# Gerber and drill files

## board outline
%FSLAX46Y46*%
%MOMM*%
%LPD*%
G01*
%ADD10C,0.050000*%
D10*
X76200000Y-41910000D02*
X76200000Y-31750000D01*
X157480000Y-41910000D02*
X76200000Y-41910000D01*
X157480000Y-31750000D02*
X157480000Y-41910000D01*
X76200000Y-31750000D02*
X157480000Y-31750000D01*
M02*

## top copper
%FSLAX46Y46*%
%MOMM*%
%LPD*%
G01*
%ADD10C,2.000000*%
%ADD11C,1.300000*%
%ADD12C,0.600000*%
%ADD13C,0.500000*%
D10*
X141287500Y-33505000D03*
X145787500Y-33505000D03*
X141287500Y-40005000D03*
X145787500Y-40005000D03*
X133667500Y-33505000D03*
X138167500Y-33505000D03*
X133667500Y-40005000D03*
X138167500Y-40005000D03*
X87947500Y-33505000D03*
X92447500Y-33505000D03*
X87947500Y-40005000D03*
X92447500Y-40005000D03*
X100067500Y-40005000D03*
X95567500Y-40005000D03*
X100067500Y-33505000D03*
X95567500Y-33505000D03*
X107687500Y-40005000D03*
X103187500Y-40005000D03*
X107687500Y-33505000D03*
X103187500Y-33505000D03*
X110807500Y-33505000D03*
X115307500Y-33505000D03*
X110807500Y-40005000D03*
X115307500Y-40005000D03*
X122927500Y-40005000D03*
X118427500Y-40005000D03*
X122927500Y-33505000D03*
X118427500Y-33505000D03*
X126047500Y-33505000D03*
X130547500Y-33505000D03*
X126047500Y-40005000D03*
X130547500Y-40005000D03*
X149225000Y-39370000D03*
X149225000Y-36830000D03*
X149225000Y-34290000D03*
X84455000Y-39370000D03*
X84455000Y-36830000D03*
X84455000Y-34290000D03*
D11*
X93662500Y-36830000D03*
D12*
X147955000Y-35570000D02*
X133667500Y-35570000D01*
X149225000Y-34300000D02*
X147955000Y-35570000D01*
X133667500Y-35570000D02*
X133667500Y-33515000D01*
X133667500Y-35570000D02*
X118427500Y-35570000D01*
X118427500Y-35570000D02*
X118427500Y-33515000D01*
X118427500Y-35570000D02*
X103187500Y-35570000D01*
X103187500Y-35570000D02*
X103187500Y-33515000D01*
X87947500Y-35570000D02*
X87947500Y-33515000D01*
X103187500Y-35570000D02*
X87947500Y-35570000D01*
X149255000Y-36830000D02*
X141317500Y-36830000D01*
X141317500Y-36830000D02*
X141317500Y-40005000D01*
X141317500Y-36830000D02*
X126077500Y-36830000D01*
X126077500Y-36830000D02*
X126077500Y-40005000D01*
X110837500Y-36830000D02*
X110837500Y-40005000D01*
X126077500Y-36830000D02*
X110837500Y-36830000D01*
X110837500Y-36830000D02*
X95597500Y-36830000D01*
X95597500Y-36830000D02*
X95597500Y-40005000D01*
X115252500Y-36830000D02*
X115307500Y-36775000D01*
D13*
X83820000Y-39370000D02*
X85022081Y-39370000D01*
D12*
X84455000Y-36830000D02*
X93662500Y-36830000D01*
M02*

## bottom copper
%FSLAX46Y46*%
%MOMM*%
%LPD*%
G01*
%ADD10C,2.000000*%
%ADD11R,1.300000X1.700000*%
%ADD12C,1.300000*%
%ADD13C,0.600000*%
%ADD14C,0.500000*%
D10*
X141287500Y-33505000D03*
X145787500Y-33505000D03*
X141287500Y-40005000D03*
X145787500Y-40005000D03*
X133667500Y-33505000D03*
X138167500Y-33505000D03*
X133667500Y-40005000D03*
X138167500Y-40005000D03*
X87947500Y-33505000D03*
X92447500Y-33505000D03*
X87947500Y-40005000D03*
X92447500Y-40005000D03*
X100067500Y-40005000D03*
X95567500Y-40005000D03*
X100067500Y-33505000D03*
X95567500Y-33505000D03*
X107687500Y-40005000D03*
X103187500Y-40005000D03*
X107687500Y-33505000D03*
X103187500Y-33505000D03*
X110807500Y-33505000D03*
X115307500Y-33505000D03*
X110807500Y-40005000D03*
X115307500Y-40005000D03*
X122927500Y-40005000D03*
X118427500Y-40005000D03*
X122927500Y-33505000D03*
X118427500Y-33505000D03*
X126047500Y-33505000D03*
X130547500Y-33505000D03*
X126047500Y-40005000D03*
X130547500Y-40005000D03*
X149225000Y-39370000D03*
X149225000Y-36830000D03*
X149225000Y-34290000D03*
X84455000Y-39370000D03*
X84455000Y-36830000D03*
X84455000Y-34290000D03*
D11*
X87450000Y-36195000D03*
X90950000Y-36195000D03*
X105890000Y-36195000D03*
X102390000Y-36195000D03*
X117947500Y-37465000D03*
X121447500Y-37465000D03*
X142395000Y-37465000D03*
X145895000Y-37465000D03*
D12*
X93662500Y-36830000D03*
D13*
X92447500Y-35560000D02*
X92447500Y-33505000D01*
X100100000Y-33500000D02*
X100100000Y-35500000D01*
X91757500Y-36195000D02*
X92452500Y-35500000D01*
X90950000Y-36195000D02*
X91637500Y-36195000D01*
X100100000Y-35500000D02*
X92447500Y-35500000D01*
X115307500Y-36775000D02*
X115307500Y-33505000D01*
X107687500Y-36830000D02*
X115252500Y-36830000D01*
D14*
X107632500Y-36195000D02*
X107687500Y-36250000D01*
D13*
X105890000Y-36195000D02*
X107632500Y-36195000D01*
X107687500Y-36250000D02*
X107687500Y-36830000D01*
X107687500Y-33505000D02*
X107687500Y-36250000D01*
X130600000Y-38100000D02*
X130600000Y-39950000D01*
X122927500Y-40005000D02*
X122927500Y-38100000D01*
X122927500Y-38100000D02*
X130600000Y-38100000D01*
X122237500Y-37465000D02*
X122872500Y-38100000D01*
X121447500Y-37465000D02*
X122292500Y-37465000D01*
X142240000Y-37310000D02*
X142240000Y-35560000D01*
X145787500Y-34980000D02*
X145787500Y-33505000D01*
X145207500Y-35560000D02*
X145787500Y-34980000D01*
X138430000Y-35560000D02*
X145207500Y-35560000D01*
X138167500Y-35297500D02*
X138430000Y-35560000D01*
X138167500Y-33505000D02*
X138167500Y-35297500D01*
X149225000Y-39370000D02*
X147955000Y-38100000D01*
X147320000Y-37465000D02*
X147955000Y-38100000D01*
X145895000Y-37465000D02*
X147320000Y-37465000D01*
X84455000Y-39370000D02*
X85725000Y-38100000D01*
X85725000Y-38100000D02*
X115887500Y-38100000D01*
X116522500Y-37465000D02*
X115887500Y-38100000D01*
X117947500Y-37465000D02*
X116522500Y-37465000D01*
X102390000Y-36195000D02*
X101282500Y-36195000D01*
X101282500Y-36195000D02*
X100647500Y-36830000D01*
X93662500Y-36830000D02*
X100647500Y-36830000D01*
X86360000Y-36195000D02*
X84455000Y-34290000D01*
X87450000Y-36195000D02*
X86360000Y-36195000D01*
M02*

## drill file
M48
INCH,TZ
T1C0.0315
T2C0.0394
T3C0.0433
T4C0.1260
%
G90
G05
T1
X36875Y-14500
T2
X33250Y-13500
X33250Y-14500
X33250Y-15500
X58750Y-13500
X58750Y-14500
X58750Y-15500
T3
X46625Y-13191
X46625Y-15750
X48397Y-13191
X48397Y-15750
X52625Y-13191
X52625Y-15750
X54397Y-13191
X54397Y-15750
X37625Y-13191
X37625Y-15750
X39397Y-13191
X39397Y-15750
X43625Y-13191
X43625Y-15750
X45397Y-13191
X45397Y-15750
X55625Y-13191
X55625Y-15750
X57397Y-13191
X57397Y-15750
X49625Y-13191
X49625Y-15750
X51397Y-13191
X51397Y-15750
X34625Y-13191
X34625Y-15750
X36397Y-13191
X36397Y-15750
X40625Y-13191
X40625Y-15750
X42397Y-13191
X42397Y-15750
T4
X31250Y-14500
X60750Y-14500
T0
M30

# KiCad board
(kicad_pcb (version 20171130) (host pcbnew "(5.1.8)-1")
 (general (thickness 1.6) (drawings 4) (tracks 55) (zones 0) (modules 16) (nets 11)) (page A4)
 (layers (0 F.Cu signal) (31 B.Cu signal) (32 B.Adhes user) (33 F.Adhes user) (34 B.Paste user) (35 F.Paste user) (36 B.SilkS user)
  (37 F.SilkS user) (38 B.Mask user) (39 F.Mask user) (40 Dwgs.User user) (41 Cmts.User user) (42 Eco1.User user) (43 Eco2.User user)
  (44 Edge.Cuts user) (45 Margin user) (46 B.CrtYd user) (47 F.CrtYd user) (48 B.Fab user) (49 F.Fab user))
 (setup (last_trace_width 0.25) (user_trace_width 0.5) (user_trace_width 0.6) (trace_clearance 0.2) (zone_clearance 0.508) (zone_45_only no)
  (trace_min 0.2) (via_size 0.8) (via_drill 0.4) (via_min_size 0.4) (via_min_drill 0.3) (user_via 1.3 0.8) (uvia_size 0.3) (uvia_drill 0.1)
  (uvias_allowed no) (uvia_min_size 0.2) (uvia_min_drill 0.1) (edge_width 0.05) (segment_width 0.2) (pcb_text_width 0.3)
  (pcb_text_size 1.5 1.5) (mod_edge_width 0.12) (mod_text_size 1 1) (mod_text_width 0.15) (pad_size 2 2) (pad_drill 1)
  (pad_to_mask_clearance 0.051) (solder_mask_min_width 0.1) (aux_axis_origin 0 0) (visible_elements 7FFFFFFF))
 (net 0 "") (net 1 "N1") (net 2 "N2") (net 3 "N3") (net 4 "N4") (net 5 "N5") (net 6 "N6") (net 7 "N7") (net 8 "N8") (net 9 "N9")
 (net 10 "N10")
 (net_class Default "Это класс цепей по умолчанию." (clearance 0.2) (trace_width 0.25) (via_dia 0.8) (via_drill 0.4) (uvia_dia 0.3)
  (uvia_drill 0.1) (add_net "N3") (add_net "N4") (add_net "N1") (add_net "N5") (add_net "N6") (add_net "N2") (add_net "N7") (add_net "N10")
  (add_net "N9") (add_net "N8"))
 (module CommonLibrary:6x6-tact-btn (layer F.Cu) (at 141.2875 40.005 90)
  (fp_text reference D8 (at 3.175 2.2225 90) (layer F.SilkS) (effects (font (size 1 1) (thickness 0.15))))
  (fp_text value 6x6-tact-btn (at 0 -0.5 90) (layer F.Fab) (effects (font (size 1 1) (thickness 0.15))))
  (pad 1 thru_hole circle (at 6.5 0 180) (size 2 2) (drill 1.1) (layers *.Cu *.Mask) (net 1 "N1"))
  (pad 2 thru_hole circle (at 6.5 4.5 180) (size 2 2) (drill 1.1) (layers *.Cu *.Mask) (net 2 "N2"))
  (pad 1 thru_hole circle (at 0 0 180) (size 2 2) (drill 1.1) (layers *.Cu *.Mask) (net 1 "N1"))
  (pad 2 thru_hole circle (at 0 4.5 180) (size 2 2) (drill 1.1) (layers *.Cu *.Mask) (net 2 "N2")))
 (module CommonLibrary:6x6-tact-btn (layer F.Cu) (at 133.6675 40.005 90)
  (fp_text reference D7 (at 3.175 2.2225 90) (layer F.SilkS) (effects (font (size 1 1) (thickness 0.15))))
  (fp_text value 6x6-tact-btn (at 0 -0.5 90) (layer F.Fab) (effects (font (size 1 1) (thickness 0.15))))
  (pad 1 thru_hole circle (at 6.5 0 180) (size 2 2) (drill 1.1) (layers *.Cu *.Mask) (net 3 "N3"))
  (pad 2 thru_hole circle (at 6.5 4.5 180) (size 2 2) (drill 1.1) (layers *.Cu *.Mask) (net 2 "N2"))
  (pad 1 thru_hole circle (at 0 0 180) (size 2 2) (drill 1.1) (layers *.Cu *.Mask) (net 3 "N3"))
  (pad 2 thru_hole circle (at 0 4.5 180) (size 2 2) (drill 1.1) (layers *.Cu *.Mask) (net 2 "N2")))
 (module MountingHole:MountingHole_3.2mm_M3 (layer F.Cu) (at 154.305 36.83)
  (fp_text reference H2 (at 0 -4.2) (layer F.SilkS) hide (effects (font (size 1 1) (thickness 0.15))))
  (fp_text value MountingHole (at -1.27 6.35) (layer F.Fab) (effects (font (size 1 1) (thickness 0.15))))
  (pad 1 np_thru_hole circle (at 0 0) (size 3.2 3.2) (drill 3.2) (layers *.Cu *.Mask)))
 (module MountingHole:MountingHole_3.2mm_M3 (layer F.Cu) (at 79.375 36.83)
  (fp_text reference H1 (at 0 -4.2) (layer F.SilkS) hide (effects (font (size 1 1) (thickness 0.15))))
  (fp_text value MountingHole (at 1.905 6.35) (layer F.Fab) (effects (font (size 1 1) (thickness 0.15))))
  (pad 1 np_thru_hole circle (at 0 0) (size 3.2 3.2) (drill 3.2) (layers *.Cu *.Mask)))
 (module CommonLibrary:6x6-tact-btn (layer F.Cu) (at 87.9475 40.005 90)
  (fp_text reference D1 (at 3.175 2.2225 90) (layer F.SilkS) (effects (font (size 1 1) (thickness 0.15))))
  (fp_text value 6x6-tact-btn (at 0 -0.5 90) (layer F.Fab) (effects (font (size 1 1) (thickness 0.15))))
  (pad 1 thru_hole circle (at 6.5 0 180) (size 2 2) (drill 1.1) (layers *.Cu *.Mask) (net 3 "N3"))
  (pad 2 thru_hole circle (at 6.5 4.5 180) (size 2 2) (drill 1.1) (layers *.Cu *.Mask) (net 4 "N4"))
  (pad 1 thru_hole circle (at 0 0 180) (size 2 2) (drill 1.1) (layers *.Cu *.Mask) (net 3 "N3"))
  (pad 2 thru_hole circle (at 0 4.5 180) (size 2 2) (drill 1.1) (layers *.Cu *.Mask) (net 4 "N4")))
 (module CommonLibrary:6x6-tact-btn (layer F.Cu) (at 95.5675 40.005 90)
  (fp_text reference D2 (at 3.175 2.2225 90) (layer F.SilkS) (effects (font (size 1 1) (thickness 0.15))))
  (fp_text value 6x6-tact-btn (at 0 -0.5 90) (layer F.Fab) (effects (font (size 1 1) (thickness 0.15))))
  (pad 2 thru_hole circle (at 0 4.5 180) (size 2 2) (drill 1.1) (layers *.Cu *.Mask) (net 4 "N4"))
  (pad 1 thru_hole circle (at 0 0 180) (size 2 2) (drill 1.1) (layers *.Cu *.Mask) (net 1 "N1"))
  (pad 2 thru_hole circle (at 6.5 4.5 180) (size 2 2) (drill 1.1) (layers *.Cu *.Mask) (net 4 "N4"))
  (pad 1 thru_hole circle (at 6.5 0 180) (size 2 2) (drill 1.1) (layers *.Cu *.Mask) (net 1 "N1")))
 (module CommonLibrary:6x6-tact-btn (layer F.Cu) (at 103.1875 40.005 90)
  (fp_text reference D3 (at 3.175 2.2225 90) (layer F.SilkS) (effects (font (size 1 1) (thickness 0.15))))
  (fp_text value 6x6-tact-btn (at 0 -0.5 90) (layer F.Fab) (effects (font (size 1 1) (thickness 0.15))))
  (pad 2 thru_hole circle (at 0 4.5 180) (size 2 2) (drill 1.1) (layers *.Cu *.Mask) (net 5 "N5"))
  (pad 1 thru_hole circle (at 0 0 180) (size 2 2) (drill 1.1) (layers *.Cu *.Mask) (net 3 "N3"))
  (pad 2 thru_hole circle (at 6.5 4.5 180) (size 2 2) (drill 1.1) (layers *.Cu *.Mask) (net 5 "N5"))
  (pad 1 thru_hole circle (at 6.5 0 180) (size 2 2) (drill 1.1) (layers *.Cu *.Mask) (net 3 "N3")))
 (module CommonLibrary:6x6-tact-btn (layer F.Cu) (at 110.8075 40.005 90)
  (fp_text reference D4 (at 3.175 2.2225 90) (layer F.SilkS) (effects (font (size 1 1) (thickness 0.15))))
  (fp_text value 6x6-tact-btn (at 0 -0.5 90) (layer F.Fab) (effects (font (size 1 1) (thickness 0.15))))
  (pad 1 thru_hole circle (at 6.5 0 180) (size 2 2) (drill 1.1) (layers *.Cu *.Mask) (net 1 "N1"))
  (pad 2 thru_hole circle (at 6.5 4.5 180) (size 2 2) (drill 1.1) (layers *.Cu *.Mask) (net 5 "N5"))
  (pad 1 thru_hole circle (at 0 0 180) (size 2 2) (drill 1.1) (layers *.Cu *.Mask) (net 1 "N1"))
  (pad 2 thru_hole circle (at 0 4.5 180) (size 2 2) (drill 1.1) (layers *.Cu *.Mask) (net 5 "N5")))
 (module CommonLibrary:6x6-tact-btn (layer F.Cu) (at 118.4275 40.005 90)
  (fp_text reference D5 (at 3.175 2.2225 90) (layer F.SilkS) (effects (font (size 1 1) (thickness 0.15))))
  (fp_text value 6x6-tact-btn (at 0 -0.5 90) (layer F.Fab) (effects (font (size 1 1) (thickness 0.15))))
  (pad 2 thru_hole circle (at 0 4.5 180) (size 2 2) (drill 1.1) (layers *.Cu *.Mask) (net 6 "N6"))
  (pad 1 thru_hole circle (at 0 0 180) (size 2 2) (drill 1.1) (layers *.Cu *.Mask) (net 3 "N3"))
  (pad 2 thru_hole circle (at 6.5 4.5 180) (size 2 2) (drill 1.1) (layers *.Cu *.Mask) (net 6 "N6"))
  (pad 1 thru_hole circle (at 6.5 0 180) (size 2 2) (drill 1.1) (layers *.Cu *.Mask) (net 3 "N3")))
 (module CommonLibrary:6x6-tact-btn (layer F.Cu) (at 126.0475 40.005 90)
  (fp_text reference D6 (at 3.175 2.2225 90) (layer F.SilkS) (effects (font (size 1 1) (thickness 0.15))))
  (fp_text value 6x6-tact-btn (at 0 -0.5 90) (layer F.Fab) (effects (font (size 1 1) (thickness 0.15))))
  (pad 1 thru_hole circle (at 6.5 0 180) (size 2 2) (drill 1.1) (layers *.Cu *.Mask) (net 1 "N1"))
  (pad 2 thru_hole circle (at 6.5 4.5 180) (size 2 2) (drill 1.1) (layers *.Cu *.Mask) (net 6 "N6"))
  (pad 1 thru_hole circle (at 0 0 180) (size 2 2) (drill 1.1) (layers *.Cu *.Mask) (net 1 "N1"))
  (pad 2 thru_hole circle (at 0 4.5 180) (size 2 2) (drill 1.1) (layers *.Cu *.Mask) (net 6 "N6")))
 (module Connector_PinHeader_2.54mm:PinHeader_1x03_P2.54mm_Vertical (layer F.Cu) (at 149.225 39.37 180)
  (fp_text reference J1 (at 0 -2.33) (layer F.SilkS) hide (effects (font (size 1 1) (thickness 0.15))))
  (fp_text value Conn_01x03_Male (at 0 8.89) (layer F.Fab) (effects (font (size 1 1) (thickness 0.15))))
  (pad 1 thru_hole circle (at 0 0 180) (size 2 2) (drill 1) (layers *.Cu *.Mask) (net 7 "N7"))
  (pad 2 thru_hole circle (at 0 2.54 180) (size 2 2) (drill 1) (layers *.Cu *.Mask) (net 1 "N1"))
  (pad 3 thru_hole circle (at 0 5.08 180) (size 2 2) (drill 1) (layers *.Cu *.Mask) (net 3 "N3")))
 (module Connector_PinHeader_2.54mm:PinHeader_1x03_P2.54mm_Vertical (layer F.Cu) (at 84.455 34.29)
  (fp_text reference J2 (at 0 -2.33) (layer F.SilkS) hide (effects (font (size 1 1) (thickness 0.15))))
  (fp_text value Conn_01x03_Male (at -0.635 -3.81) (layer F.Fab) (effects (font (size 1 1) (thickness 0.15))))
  (pad 3 thru_hole circle (at 0 5.08) (size 2 2) (drill 1) (layers *.Cu *.Mask) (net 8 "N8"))
  (pad 2 thru_hole circle (at 0 2.54) (size 2 2) (drill 1) (layers *.Cu *.Mask) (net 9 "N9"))
  (pad 1 thru_hole circle (at 0 0) (size 2 2) (drill 1) (layers *.Cu *.Mask) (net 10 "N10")))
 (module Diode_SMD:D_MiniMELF (layer B.Cu) (at 89.2 36.195)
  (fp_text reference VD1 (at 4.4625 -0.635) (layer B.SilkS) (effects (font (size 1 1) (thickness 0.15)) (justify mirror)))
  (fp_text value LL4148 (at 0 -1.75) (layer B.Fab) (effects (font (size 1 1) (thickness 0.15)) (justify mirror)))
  (pad 1 smd rect (at -1.75 0) (size 1.3 1.7) (layers B.Cu B.Paste B.Mask) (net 10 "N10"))
  (pad 2 smd rect (at 1.75 0) (size 1.3 1.7) (layers B.Cu B.Paste B.Mask) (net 4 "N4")))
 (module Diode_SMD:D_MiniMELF (layer B.Cu) (at 104.14 36.195)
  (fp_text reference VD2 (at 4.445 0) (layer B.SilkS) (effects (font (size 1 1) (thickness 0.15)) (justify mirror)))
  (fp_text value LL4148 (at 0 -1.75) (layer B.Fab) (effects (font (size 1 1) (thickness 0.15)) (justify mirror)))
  (pad 2 smd rect (at 1.75 0) (size 1.3 1.7) (layers B.Cu B.Paste B.Mask) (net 5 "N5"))
  (pad 1 smd rect (at -1.75 0) (size 1.3 1.7) (layers B.Cu B.Paste B.Mask) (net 9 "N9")))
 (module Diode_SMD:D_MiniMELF (layer B.Cu) (at 119.6975 37.465)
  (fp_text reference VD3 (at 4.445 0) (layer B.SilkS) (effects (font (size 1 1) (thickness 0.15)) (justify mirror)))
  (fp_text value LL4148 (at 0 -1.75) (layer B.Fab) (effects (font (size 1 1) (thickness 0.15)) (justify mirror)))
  (pad 1 smd rect (at -1.75 0) (size 1.3 1.7) (layers B.Cu B.Paste B.Mask) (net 8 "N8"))
  (pad 2 smd rect (at 1.75 0) (size 1.3 1.7) (layers B.Cu B.Paste B.Mask) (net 6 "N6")))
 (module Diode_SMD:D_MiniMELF (layer B.Cu) (at 144.145 37.465 180)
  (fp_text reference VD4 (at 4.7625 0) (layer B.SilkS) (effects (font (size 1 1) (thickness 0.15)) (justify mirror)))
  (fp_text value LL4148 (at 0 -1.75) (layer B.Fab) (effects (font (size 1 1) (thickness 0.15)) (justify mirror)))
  (pad 2 smd rect (at 1.75 0 180) (size 1.3 1.7) (layers B.Cu B.Paste B.Mask) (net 2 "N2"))
  (pad 1 smd rect (at -1.75 0 180) (size 1.3 1.7) (layers B.Cu B.Paste B.Mask) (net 7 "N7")))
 (gr_line (start 76.2 41.91) (end 76.2 31.75) (layer Edge.Cuts) (width 0.05))
 (gr_line (start 157.48 41.91) (end 76.2 41.91) (layer Edge.Cuts) (width 0.05))
 (gr_line (start 157.48 31.75) (end 157.48 41.91) (layer Edge.Cuts) (width 0.05))
 (gr_line (start 76.2 31.75) (end 157.48 31.75) (layer Edge.Cuts) (width 0.05))
 (segment (start 147.955 35.57) (end 133.6675 35.57) (width 0.6) (layer F.Cu) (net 3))
 (segment (start 149.225 34.3) (end 147.955 35.57) (width 0.6) (layer F.Cu) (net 3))
 (segment (start 133.6675 35.57) (end 133.6675 33.515) (width 0.6) (layer F.Cu) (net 3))
 (segment (start 133.6675 35.57) (end 118.4275 35.57) (width 0.6) (layer F.Cu) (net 3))
 (segment (start 118.4275 35.57) (end 118.4275 33.515) (width 0.6) (layer F.Cu) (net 3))
 (segment (start 118.4275 35.57) (end 103.1875 35.57) (width 0.6) (layer F.Cu) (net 3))
 (segment (start 103.1875 35.57) (end 103.1875 33.515) (width 0.6) (layer F.Cu) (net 3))
 (segment (start 87.9475 35.57) (end 87.9475 33.515) (width 0.6) (layer F.Cu) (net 3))
 (segment (start 103.1875 35.57) (end 87.9475 35.57) (width 0.6) (layer F.Cu) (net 3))
 (segment (start 92.4475 35.56) (end 92.4475 33.505) (width 0.6) (layer B.Cu) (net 4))
 (segment (start 100.1 33.5) (end 100.1 35.5) (width 0.6) (layer B.Cu) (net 4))
 (segment (start 91.7575 36.195) (end 92.4525 35.5) (width 0.6) (layer B.Cu) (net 4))
 (segment (start 90.95 36.195) (end 91.6375 36.195) (width 0.6) (layer B.Cu) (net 4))
 (segment (start 100.1 35.5) (end 92.4475 35.5) (width 0.6) (layer B.Cu) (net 4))
 (segment (start 149.255 36.83) (end 141.3175 36.83) (width 0.6) (layer F.Cu) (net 1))
 (segment (start 141.3175 36.83) (end 141.3175 40.005) (width 0.6) (layer F.Cu) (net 1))
 (segment (start 141.3175 36.83) (end 126.0775 36.83) (width 0.6) (layer F.Cu) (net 1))
 (segment (start 126.0775 36.83) (end 126.0775 40.005) (width 0.6) (layer F.Cu) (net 1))
 (segment (start 110.8375 36.83) (end 110.8375 40.005) (width 0.6) (layer F.Cu) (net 1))
 (segment (start 126.0775 36.83) (end 110.8375 36.83) (width 0.6) (layer F.Cu) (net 1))
 (segment (start 110.8375 36.83) (end 95.5975 36.83) (width 0.6) (layer F.Cu) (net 1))
 (segment (start 95.5975 36.83) (end 95.5975 40.005) (width 0.6) (layer F.Cu) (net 1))
 (segment (start 115.2525 36.83) (end 115.3075 36.775) (width 0.6) (layer F.Cu) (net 1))
 (segment (start 115.3075 36.775) (end 115.3075 33.505) (width 0.6) (layer B.Cu) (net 5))
 (segment (start 107.6875 36.83) (end 115.2525 36.83) (width 0.6) (layer B.Cu) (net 5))
 (segment (start 107.6325 36.195) (end 107.6875 36.25) (width 0.5) (layer B.Cu) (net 5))
 (segment (start 105.89 36.195) (end 107.6325 36.195) (width 0.6) (layer B.Cu) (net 5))
 (segment (start 107.6875 36.25) (end 107.6875 36.83) (width 0.6) (layer B.Cu) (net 5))
 (segment (start 107.6875 33.505) (end 107.6875 36.25) (width 0.6) (layer B.Cu) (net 5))
 (segment (start 130.6 38.1) (end 130.6 39.95) (width 0.6) (layer B.Cu) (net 6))
 (segment (start 122.9275 40.005) (end 122.9275 38.1) (width 0.6) (layer B.Cu) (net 6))
 (segment (start 122.9275 38.1) (end 130.6 38.1) (width 0.6) (layer B.Cu) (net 6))
 (segment (start 122.2375 37.465) (end 122.8725 38.1) (width 0.6) (layer B.Cu) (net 6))
 (segment (start 121.4475 37.465) (end 122.2925 37.465) (width 0.6) (layer B.Cu) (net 6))
 (segment (start 142.24 37.31) (end 142.24 35.56) (width 0.6) (layer B.Cu) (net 2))
 (segment (start 145.7875 34.98) (end 145.7875 33.505) (width 0.6) (layer B.Cu) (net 2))
 (segment (start 145.2075 35.56) (end 145.7875 34.98) (width 0.6) (layer B.Cu) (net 2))
 (segment (start 138.43 35.56) (end 145.2075 35.56) (width 0.6) (layer B.Cu) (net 2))
 (segment (start 138.1675 35.2975) (end 138.43 35.56) (width 0.6) (layer B.Cu) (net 2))
 (segment (start 138.1675 33.505) (end 138.1675 35.2975) (width 0.6) (layer B.Cu) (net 2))
 (segment (start 149.225 39.37) (end 147.955 38.1) (width 0.6) (layer B.Cu) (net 7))
 (segment (start 147.32 37.465) (end 147.955 38.1) (width 0.6) (layer B.Cu) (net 7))
 (segment (start 145.895 37.465) (end 147.32 37.465) (width 0.6) (layer B.Cu) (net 7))
 (segment (start 83.82 39.37) (end 85.022081 39.37) (width 0.5) (layer F.Cu) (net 8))
 (segment (start 84.455 39.37) (end 85.725 38.1) (width 0.6) (layer B.Cu) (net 8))
 (segment (start 85.725 38.1) (end 115.8875 38.1) (width 0.6) (layer B.Cu) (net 8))
 (segment (start 116.5225 37.465) (end 115.8875 38.1) (width 0.6) (layer B.Cu) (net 8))
 (segment (start 117.9475 37.465) (end 116.5225 37.465) (width 0.6) (layer B.Cu) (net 8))
 (segment (start 84.455 36.83) (end 93.6625 36.83) (width 0.6) (layer F.Cu) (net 9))
 (via (at 93.6625 36.83) (size 1.3) (drill 0.8) (layers F.Cu B.Cu) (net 9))
 (segment (start 102.39 36.195) (end 101.2825 36.195) (width 0.6) (layer B.Cu) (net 9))
 (segment (start 101.2825 36.195) (end 100.6475 36.83) (width 0.6) (layer B.Cu) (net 9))
 (segment (start 93.6625 36.83) (end 100.6475 36.83) (width 0.6) (layer B.Cu) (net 9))
 (segment (start 86.36 36.195) (end 84.455 34.29) (width 0.6) (layer B.Cu) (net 10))
 (segment (start 87.45 36.195) (end 86.36 36.195) (width 0.6) (layer B.Cu) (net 10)))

